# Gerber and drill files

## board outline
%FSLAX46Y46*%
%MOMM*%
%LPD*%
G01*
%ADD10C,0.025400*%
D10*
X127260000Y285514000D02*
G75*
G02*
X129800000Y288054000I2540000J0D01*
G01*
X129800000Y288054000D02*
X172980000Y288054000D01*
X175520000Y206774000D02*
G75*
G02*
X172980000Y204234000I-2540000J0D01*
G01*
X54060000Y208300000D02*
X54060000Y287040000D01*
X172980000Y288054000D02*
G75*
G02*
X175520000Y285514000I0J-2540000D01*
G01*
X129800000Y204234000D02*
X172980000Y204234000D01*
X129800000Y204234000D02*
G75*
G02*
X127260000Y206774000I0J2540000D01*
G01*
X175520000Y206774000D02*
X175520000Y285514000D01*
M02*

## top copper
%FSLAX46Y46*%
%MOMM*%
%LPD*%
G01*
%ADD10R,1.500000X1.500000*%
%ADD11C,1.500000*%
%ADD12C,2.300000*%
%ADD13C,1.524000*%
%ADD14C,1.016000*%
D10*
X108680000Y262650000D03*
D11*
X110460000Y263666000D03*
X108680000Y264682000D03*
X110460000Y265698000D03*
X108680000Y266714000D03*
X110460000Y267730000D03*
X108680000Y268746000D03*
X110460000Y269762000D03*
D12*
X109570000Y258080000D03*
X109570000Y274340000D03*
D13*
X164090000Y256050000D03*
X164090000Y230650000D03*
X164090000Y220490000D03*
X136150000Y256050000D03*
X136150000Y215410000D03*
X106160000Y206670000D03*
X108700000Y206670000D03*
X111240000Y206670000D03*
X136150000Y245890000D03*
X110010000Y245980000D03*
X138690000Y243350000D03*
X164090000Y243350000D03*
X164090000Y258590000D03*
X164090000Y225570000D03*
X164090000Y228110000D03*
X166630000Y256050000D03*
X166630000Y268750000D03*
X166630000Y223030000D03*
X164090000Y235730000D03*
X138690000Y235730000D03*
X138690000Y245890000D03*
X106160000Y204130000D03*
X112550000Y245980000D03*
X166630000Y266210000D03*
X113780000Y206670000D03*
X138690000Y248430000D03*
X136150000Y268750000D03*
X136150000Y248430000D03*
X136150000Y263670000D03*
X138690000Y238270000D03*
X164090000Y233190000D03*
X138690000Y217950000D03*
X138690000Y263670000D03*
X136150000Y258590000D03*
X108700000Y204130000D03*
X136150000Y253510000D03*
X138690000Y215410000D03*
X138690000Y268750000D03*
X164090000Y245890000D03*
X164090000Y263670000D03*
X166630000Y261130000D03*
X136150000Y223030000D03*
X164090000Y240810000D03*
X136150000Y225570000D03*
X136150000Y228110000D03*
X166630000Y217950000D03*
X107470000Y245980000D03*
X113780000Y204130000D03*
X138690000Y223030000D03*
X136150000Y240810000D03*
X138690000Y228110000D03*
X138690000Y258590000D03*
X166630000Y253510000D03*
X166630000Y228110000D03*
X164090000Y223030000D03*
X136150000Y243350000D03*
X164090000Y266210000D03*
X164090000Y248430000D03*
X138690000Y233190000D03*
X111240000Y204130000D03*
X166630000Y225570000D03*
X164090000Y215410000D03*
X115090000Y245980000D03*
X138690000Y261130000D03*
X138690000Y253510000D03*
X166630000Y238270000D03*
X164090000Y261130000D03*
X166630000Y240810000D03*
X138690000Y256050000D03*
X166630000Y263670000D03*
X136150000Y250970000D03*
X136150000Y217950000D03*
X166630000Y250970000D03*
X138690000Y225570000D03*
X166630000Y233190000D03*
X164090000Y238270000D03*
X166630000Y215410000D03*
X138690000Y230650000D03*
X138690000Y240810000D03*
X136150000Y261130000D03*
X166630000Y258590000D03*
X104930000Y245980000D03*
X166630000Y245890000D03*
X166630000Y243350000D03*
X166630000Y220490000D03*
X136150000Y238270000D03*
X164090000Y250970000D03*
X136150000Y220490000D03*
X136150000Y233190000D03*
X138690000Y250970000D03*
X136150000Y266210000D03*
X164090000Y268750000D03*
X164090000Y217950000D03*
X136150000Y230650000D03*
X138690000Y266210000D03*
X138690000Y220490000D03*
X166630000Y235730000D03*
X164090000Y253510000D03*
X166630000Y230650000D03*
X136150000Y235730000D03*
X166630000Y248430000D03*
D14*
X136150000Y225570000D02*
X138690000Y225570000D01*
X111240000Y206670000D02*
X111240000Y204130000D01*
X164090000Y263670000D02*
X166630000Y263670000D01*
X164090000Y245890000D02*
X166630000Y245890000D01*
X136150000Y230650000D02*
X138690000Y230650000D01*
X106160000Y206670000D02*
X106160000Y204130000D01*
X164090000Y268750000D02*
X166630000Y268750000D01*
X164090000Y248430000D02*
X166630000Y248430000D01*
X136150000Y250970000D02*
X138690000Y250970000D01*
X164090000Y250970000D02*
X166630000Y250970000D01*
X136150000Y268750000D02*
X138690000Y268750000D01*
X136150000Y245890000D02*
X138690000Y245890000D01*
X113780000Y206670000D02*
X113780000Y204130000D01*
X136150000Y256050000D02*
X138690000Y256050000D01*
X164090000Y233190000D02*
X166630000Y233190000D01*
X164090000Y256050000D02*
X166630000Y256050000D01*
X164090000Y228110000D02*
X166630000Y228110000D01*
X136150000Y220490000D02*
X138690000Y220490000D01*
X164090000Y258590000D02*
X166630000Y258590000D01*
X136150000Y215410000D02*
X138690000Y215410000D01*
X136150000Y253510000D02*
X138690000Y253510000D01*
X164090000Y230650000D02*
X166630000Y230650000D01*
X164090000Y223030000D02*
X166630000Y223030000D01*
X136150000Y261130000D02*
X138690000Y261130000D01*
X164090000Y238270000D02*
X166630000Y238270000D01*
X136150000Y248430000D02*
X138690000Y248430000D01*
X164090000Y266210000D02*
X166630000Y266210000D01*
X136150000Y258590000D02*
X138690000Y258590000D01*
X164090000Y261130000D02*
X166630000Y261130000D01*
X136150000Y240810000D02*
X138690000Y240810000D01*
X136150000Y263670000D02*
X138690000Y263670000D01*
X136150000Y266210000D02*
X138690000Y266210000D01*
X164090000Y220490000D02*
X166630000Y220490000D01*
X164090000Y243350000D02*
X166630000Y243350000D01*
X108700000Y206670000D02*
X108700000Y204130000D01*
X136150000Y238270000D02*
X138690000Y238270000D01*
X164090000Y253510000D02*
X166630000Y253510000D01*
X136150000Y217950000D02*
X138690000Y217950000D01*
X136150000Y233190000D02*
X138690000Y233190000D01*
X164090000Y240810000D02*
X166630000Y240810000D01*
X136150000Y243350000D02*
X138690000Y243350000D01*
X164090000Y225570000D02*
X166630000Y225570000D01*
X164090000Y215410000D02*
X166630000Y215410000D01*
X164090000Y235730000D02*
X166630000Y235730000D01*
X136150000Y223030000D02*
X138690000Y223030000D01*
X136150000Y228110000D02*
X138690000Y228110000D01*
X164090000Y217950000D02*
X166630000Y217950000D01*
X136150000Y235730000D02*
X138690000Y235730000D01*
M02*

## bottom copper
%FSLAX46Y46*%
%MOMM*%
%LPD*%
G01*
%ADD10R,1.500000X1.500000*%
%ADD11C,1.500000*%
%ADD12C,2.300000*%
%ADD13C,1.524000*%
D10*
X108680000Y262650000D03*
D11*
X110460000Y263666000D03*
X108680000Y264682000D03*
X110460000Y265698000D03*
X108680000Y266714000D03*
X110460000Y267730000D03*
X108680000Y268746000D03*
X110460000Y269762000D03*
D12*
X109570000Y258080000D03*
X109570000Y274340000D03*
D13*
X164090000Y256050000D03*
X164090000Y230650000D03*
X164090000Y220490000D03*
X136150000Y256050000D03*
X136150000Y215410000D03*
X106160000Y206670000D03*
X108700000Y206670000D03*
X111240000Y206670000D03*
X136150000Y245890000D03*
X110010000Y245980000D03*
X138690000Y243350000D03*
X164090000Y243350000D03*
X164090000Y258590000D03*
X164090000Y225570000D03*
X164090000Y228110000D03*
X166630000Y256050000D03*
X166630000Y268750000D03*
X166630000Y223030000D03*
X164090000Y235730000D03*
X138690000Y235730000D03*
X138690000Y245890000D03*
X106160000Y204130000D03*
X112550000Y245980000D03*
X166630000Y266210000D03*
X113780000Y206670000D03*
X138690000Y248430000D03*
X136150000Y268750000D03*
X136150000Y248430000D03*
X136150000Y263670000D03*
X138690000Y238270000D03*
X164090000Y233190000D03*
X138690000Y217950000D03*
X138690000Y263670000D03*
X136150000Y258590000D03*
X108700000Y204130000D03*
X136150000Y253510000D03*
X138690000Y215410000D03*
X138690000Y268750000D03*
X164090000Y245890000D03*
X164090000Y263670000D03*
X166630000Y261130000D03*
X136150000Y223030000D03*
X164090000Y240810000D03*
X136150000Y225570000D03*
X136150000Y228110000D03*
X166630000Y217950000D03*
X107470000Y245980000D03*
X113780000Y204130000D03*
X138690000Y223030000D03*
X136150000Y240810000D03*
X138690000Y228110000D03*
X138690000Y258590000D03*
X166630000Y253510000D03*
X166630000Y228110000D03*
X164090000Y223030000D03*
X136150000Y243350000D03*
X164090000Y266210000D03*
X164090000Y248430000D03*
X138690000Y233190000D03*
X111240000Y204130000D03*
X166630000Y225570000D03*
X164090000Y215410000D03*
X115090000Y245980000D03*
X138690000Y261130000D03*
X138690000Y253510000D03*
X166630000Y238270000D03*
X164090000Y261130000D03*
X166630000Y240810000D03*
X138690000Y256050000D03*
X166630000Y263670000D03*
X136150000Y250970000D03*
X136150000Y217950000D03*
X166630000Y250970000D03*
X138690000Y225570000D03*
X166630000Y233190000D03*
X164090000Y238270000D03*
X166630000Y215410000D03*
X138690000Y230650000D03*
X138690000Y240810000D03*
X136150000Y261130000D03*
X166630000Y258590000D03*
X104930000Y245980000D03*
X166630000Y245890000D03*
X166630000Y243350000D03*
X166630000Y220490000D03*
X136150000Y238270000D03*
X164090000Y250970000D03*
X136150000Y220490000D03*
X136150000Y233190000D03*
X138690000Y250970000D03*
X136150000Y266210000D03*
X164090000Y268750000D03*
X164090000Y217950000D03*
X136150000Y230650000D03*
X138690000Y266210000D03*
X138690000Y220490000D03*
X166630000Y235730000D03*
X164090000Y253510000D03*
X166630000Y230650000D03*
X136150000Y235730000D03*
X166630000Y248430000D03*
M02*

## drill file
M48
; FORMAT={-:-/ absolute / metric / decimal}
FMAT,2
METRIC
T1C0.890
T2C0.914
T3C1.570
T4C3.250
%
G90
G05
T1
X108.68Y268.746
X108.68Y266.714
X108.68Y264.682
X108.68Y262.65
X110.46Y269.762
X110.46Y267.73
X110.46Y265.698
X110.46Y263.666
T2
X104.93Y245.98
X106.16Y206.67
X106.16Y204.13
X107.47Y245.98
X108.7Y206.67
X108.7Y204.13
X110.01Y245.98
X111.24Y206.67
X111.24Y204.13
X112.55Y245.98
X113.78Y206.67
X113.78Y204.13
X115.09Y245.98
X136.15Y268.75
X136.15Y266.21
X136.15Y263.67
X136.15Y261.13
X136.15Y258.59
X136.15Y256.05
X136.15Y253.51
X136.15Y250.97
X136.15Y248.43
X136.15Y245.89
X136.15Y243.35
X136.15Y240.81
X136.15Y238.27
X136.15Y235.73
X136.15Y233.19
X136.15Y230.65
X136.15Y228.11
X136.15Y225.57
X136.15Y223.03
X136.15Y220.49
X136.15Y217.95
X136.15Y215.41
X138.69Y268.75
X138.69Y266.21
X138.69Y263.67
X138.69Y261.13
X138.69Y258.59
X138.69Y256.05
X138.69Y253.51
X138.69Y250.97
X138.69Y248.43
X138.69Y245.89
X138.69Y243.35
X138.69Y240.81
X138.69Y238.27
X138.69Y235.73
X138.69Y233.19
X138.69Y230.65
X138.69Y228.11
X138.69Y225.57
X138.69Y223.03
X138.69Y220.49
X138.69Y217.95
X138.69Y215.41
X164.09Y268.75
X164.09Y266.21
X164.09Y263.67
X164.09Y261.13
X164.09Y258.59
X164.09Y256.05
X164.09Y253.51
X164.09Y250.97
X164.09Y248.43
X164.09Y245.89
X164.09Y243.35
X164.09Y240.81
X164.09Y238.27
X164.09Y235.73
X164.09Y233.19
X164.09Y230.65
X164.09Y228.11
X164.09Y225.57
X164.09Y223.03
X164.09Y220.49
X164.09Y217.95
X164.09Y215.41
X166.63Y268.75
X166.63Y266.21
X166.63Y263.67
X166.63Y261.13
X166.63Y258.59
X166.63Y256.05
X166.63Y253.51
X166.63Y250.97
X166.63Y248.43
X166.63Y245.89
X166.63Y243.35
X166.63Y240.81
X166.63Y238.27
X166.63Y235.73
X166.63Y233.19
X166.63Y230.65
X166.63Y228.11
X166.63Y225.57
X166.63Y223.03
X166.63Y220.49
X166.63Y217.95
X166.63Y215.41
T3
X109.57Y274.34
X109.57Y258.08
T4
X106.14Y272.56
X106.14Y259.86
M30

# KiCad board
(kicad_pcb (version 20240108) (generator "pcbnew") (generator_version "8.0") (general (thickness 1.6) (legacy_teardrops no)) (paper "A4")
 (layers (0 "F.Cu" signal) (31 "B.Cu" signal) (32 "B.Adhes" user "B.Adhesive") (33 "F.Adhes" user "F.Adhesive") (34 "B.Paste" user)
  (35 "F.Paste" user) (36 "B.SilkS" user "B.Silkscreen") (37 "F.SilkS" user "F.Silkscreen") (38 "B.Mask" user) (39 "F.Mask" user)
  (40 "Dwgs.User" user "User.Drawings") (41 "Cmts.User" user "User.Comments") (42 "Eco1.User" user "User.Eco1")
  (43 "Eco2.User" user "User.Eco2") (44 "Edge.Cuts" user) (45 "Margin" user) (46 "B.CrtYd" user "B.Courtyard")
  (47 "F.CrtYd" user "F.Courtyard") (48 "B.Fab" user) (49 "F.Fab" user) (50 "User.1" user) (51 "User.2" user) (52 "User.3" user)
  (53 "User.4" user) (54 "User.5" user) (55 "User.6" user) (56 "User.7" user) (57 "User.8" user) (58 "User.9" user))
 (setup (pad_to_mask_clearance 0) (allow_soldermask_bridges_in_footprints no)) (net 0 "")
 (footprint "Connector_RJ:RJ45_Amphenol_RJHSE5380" (layer "F.Cu") (at 108.68 -262.65 90)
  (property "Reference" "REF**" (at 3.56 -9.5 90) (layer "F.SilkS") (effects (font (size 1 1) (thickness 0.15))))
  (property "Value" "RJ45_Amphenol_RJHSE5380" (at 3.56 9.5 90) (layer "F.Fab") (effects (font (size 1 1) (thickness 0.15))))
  (pad "" np_thru_hole circle (at -2.79 -2.54 90) (size 3.25 3.25) (drill 3.25) (layers "*.Cu" "*.Mask"))
  (pad "" np_thru_hole circle (at 9.91 -2.54 90) (size 3.25 3.25) (drill 3.25) (layers "*.Cu" "*.Mask"))
  (pad "1" thru_hole rect (at 0 0 90) (size 1.5 1.5) (drill 0.89) (layers "*.Cu" "*.Mask") (remove_unused_layers no))
  (pad "2" thru_hole circle (at 1.016 1.78 90) (size 1.5 1.5) (drill 0.89) (layers "*.Cu" "*.Mask") (remove_unused_layers no))
  (pad "3" thru_hole circle (at 2.032 0 90) (size 1.5 1.5) (drill 0.89) (layers "*.Cu" "*.Mask") (remove_unused_layers no))
  (pad "4" thru_hole circle (at 3.048 1.78 90) (size 1.5 1.5) (drill 0.89) (layers "*.Cu" "*.Mask") (remove_unused_layers no))
  (pad "5" thru_hole circle (at 4.064 0 90) (size 1.5 1.5) (drill 0.89) (layers "*.Cu" "*.Mask") (remove_unused_layers no))
  (pad "6" thru_hole circle (at 5.08 1.78 90) (size 1.5 1.5) (drill 0.89) (layers "*.Cu" "*.Mask") (remove_unused_layers no))
  (pad "7" thru_hole circle (at 6.096 0 90) (size 1.5 1.5) (drill 0.89) (layers "*.Cu" "*.Mask") (remove_unused_layers no))
  (pad "8" thru_hole circle (at 7.112 1.78 90) (size 1.5 1.5) (drill 0.89) (layers "*.Cu" "*.Mask") (remove_unused_layers no))
  (pad "SH" thru_hole circle (at -4.57 0.89 90) (size 2.3 2.3) (drill 1.57) (layers "*.Cu" "*.Mask") (remove_unused_layers no))
  (pad "SH" thru_hole circle (at 11.69 0.89 90) (size 2.3 2.3) (drill 1.57) (layers "*.Cu" "*.Mask") (remove_unused_layers no)))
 (gr_arc (start 127.26 -285.514) (mid 128.003949 -287.310051) (end 129.8 -288.054) (stroke (width 0.0254) (type default))
  (layer "Edge.Cuts"))
 (gr_line (start 129.8 -288.054) (end 172.98 -288.054) (stroke (width 0.0254) (type default)) (layer "Edge.Cuts"))
 (gr_arc (start 175.52 -206.774) (mid 174.776051 -204.977949) (end 172.98 -204.234) (stroke (width 0.0254) (type default))
  (layer "Edge.Cuts"))
 (gr_line (start 54.06 -208.3) (end 54.06 -287.04) (stroke (width 0.0254) (type solid)) (layer "Edge.Cuts"))
 (gr_arc (start 172.98 -288.054) (mid 174.776051 -287.310051) (end 175.52 -285.514) (stroke (width 0.0254) (type default))
  (layer "Edge.Cuts"))
 (gr_line (start 129.8 -204.234) (end 172.98 -204.234) (stroke (width 0.0254) (type default)) (layer "Edge.Cuts"))
 (gr_arc (start 129.8 -204.234) (mid 128.003949 -204.977949) (end 127.26 -206.774) (stroke (width 0.0254) (type default))
  (layer "Edge.Cuts"))
 (gr_line (start 175.52 -206.774) (end 175.52 -285.514) (stroke (width 0.0254) (type solid)) (layer "Edge.Cuts"))
 (segment (start 136.15 -225.57) (end 138.69 -225.57) (width 1.016) (layer "F.Cu") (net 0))
 (segment (start 111.24 -206.67) (end 111.24 -204.13) (width 1.016) (layer "F.Cu") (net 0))
 (segment (start 164.09 -263.67) (end 166.63 -263.67) (width 1.016) (layer "F.Cu") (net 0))
 (segment (start 164.09 -245.89) (end 166.63 -245.89) (width 1.016) (layer "F.Cu") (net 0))
 (segment (start 136.15 -230.65) (end 138.69 -230.65) (width 1.016) (layer "F.Cu") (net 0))
 (segment (start 106.16 -206.67) (end 106.16 -204.13) (width 1.016) (layer "F.Cu") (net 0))
 (segment (start 164.09 -268.75) (end 166.63 -268.75) (width 1.016) (layer "F.Cu") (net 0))
 (segment (start 164.09 -248.43) (end 166.63 -248.43) (width 1.016) (layer "F.Cu") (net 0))
 (segment (start 136.15 -250.97) (end 138.69 -250.97) (width 1.016) (layer "F.Cu") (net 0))
 (segment (start 164.09 -250.97) (end 166.63 -250.97) (width 1.016) (layer "F.Cu") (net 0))
 (segment (start 136.15 -268.75) (end 138.69 -268.75) (width 1.016) (layer "F.Cu") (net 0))
 (segment (start 136.15 -245.89) (end 138.69 -245.89) (width 1.016) (layer "F.Cu") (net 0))
 (segment (start 113.78 -206.67) (end 113.78 -204.13) (width 1.016) (layer "F.Cu") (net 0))
 (segment (start 136.15 -256.05) (end 138.69 -256.05) (width 1.016) (layer "F.Cu") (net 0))
 (segment (start 164.09 -233.19) (end 166.63 -233.19) (width 1.016) (layer "F.Cu") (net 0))
 (segment (start 164.09 -256.05) (end 166.63 -256.05) (width 1.016) (layer "F.Cu") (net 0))
 (segment (start 164.09 -228.11) (end 166.63 -228.11) (width 1.016) (layer "F.Cu") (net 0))
 (segment (start 136.15 -220.49) (end 138.69 -220.49) (width 1.016) (layer "F.Cu") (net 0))
 (segment (start 164.09 -258.59) (end 166.63 -258.59) (width 1.016) (layer "F.Cu") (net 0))
 (segment (start 136.15 -215.41) (end 138.69 -215.41) (width 1.016) (layer "F.Cu") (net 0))
 (segment (start 136.15 -253.51) (end 138.69 -253.51) (width 1.016) (layer "F.Cu") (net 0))
 (segment (start 164.09 -230.65) (end 166.63 -230.65) (width 1.016) (layer "F.Cu") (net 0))
 (segment (start 164.09 -223.03) (end 166.63 -223.03) (width 1.016) (layer "F.Cu") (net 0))
 (segment (start 136.15 -261.13) (end 138.69 -261.13) (width 1.016) (layer "F.Cu") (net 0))
 (segment (start 164.09 -238.27) (end 166.63 -238.27) (width 1.016) (layer "F.Cu") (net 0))
 (segment (start 136.15 -248.43) (end 138.69 -248.43) (width 1.016) (layer "F.Cu") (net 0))
 (segment (start 164.09 -266.21) (end 166.63 -266.21) (width 1.016) (layer "F.Cu") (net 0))
 (segment (start 136.15 -258.59) (end 138.69 -258.59) (width 1.016) (layer "F.Cu") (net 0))
 (segment (start 164.09 -261.13) (end 166.63 -261.13) (width 1.016) (layer "F.Cu") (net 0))
 (segment (start 136.15 -240.81) (end 138.69 -240.81) (width 1.016) (layer "F.Cu") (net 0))
 (segment (start 136.15 -263.67) (end 138.69 -263.67) (width 1.016) (layer "F.Cu") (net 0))
 (segment (start 136.15 -266.21) (end 138.69 -266.21) (width 1.016) (layer "F.Cu") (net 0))
 (segment (start 164.09 -220.49) (end 166.63 -220.49) (width 1.016) (layer "F.Cu") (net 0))
 (segment (start 164.09 -243.35) (end 166.63 -243.35) (width 1.016) (layer "F.Cu") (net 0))
 (segment (start 108.7 -206.67) (end 108.7 -204.13) (width 1.016) (layer "F.Cu") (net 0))
 (segment (start 136.15 -238.27) (end 138.69 -238.27) (width 1.016) (layer "F.Cu") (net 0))
 (segment (start 164.09 -253.51) (end 166.63 -253.51) (width 1.016) (layer "F.Cu") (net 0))
 (segment (start 136.15 -217.95) (end 138.69 -217.95) (width 1.016) (layer "F.Cu") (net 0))
 (segment (start 136.15 -233.19) (end 138.69 -233.19) (width 1.016) (layer "F.Cu") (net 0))
 (segment (start 164.09 -240.81) (end 166.63 -240.81) (width 1.016) (layer "F.Cu") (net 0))
 (segment (start 136.15 -243.35) (end 138.69 -243.35) (width 1.016) (layer "F.Cu") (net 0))
 (segment (start 164.09 -225.57) (end 166.63 -225.57) (width 1.016) (layer "F.Cu") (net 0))
 (segment (start 164.09 -215.41) (end 166.63 -215.41) (width 1.016) (layer "F.Cu") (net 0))
 (segment (start 164.09 -235.73) (end 166.63 -235.73) (width 1.016) (layer "F.Cu") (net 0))
 (segment (start 136.15 -223.03) (end 138.69 -223.03) (width 1.016) (layer "F.Cu") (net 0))
 (segment (start 136.15 -228.11) (end 138.69 -228.11) (width 1.016) (layer "F.Cu") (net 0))
 (segment (start 164.09 -217.95) (end 166.63 -217.95) (width 1.016) (layer "F.Cu") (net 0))
 (segment (start 136.15 -235.73) (end 138.69 -235.73) (width 1.016) (layer "F.Cu") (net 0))
 (via (at 164.09 -256.05) (size 1.524) (drill 0.9144) (layers "F.Cu" "B.Cu") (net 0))
 (via (at 164.09 -230.65) (size 1.524) (drill 0.9144) (layers "F.Cu" "B.Cu") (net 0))
 (via (at 164.09 -220.49) (size 1.524) (drill 0.9144) (layers "F.Cu" "B.Cu") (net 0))
 (via (at 136.15 -256.05) (size 1.524) (drill 0.9144) (layers "F.Cu" "B.Cu") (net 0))
 (via (at 136.15 -215.41) (size 1.524) (drill 0.9144) (layers "F.Cu" "B.Cu") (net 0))
 (via (at 106.16 -206.67) (size 1.524) (drill 0.9144) (layers "F.Cu" "B.Cu") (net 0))
 (via (at 108.7 -206.67) (size 1.524) (drill 0.9144) (layers "F.Cu" "B.Cu") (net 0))
 (via (at 111.24 -206.67) (size 1.524) (drill 0.9144) (layers "F.Cu" "B.Cu") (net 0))
 (via (at 136.15 -245.89) (size 1.524) (drill 0.9144) (layers "F.Cu" "B.Cu") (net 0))
 (via (at 110.01 -245.98) (size 1.524) (drill 0.9144) (layers "F.Cu" "B.Cu") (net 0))
 (via (at 138.69 -243.35) (size 1.524) (drill 0.9144) (layers "F.Cu" "B.Cu") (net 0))
 (via (at 164.09 -243.35) (size 1.524) (drill 0.9144) (layers "F.Cu" "B.Cu") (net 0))
 (via (at 164.09 -258.59) (size 1.524) (drill 0.9144) (layers "F.Cu" "B.Cu") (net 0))
 (via (at 164.09 -225.57) (size 1.524) (drill 0.9144) (layers "F.Cu" "B.Cu") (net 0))
 (via (at 164.09 -228.11) (size 1.524) (drill 0.9144) (layers "F.Cu" "B.Cu") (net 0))
 (via (at 166.63 -256.05) (size 1.524) (drill 0.9144) (layers "F.Cu" "B.Cu") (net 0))
 (via (at 166.63 -268.75) (size 1.524) (drill 0.9144) (layers "F.Cu" "B.Cu") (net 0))
 (via (at 166.63 -223.03) (size 1.524) (drill 0.9144) (layers "F.Cu" "B.Cu") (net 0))
 (via (at 164.09 -235.73) (size 1.524) (drill 0.9144) (layers "F.Cu" "B.Cu") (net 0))
 (via (at 138.69 -235.73) (size 1.524) (drill 0.9144) (layers "F.Cu" "B.Cu") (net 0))
 (via (at 138.69 -245.89) (size 1.524) (drill 0.9144) (layers "F.Cu" "B.Cu") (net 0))
 (via (at 106.16 -204.13) (size 1.524) (drill 0.9144) (layers "F.Cu" "B.Cu") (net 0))
 (via (at 112.55 -245.98) (size 1.524) (drill 0.9144) (layers "F.Cu" "B.Cu") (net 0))
 (via (at 166.63 -266.21) (size 1.524) (drill 0.9144) (layers "F.Cu" "B.Cu") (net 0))
 (via (at 113.78 -206.67) (size 1.524) (drill 0.9144) (layers "F.Cu" "B.Cu") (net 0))
 (via (at 138.69 -248.43) (size 1.524) (drill 0.9144) (layers "F.Cu" "B.Cu") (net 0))
 (via (at 136.15 -268.75) (size 1.524) (drill 0.9144) (layers "F.Cu" "B.Cu") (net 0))
 (via (at 136.15 -248.43) (size 1.524) (drill 0.9144) (layers "F.Cu" "B.Cu") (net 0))
 (via (at 136.15 -263.67) (size 1.524) (drill 0.9144) (layers "F.Cu" "B.Cu") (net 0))
 (via (at 138.69 -238.27) (size 1.524) (drill 0.9144) (layers "F.Cu" "B.Cu") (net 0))
 (via (at 164.09 -233.19) (size 1.524) (drill 0.9144) (layers "F.Cu" "B.Cu") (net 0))
 (via (at 138.69 -217.95) (size 1.524) (drill 0.9144) (layers "F.Cu" "B.Cu") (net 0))
 (via (at 138.69 -263.67) (size 1.524) (drill 0.9144) (layers "F.Cu" "B.Cu") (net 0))
 (via (at 136.15 -258.59) (size 1.524) (drill 0.9144) (layers "F.Cu" "B.Cu") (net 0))
 (via (at 108.7 -204.13) (size 1.524) (drill 0.9144) (layers "F.Cu" "B.Cu") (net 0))
 (via (at 136.15 -253.51) (size 1.524) (drill 0.9144) (layers "F.Cu" "B.Cu") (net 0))
 (via (at 138.69 -215.41) (size 1.524) (drill 0.9144) (layers "F.Cu" "B.Cu") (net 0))
 (via (at 138.69 -268.75) (size 1.524) (drill 0.9144) (layers "F.Cu" "B.Cu") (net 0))
 (via (at 164.09 -245.89) (size 1.524) (drill 0.9144) (layers "F.Cu" "B.Cu") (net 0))
 (via (at 164.09 -263.67) (size 1.524) (drill 0.9144) (layers "F.Cu" "B.Cu") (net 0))
 (via (at 166.63 -261.13) (size 1.524) (drill 0.9144) (layers "F.Cu" "B.Cu") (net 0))
 (via (at 136.15 -223.03) (size 1.524) (drill 0.9144) (layers "F.Cu" "B.Cu") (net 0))
 (via (at 164.09 -240.81) (size 1.524) (drill 0.9144) (layers "F.Cu" "B.Cu") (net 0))
 (via (at 136.15 -225.57) (size 1.524) (drill 0.9144) (layers "F.Cu" "B.Cu") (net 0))
 (via (at 136.15 -228.11) (size 1.524) (drill 0.9144) (layers "F.Cu" "B.Cu") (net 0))
 (via (at 166.63 -217.95) (size 1.524) (drill 0.9144) (layers "F.Cu" "B.Cu") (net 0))
 (via (at 107.47 -245.98) (size 1.524) (drill 0.9144) (layers "F.Cu" "B.Cu") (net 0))
 (via (at 113.78 -204.13) (size 1.524) (drill 0.9144) (layers "F.Cu" "B.Cu") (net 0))
 (via (at 138.69 -223.03) (size 1.524) (drill 0.9144) (layers "F.Cu" "B.Cu") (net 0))
 (via (at 136.15 -240.81) (size 1.524) (drill 0.9144) (layers "F.Cu" "B.Cu") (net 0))
 (via (at 138.69 -228.11) (size 1.524) (drill 0.9144) (layers "F.Cu" "B.Cu") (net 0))
 (via (at 138.69 -258.59) (size 1.524) (drill 0.9144) (layers "F.Cu" "B.Cu") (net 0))
 (via (at 166.63 -253.51) (size 1.524) (drill 0.9144) (layers "F.Cu" "B.Cu") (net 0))
 (via (at 166.63 -228.11) (size 1.524) (drill 0.9144) (layers "F.Cu" "B.Cu") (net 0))
 (via (at 164.09 -223.03) (size 1.524) (drill 0.9144) (layers "F.Cu" "B.Cu") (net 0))
 (via (at 136.15 -243.35) (size 1.524) (drill 0.9144) (layers "F.Cu" "B.Cu") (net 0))
 (via (at 164.09 -266.21) (size 1.524) (drill 0.9144) (layers "F.Cu" "B.Cu") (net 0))
 (via (at 164.09 -248.43) (size 1.524) (drill 0.9144) (layers "F.Cu" "B.Cu") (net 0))
 (via (at 138.69 -233.19) (size 1.524) (drill 0.9144) (layers "F.Cu" "B.Cu") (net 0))
 (via (at 111.24 -204.13) (size 1.524) (drill 0.9144) (layers "F.Cu" "B.Cu") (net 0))
 (via (at 166.63 -225.57) (size 1.524) (drill 0.9144) (layers "F.Cu" "B.Cu") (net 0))
 (via (at 164.09 -215.41) (size 1.524) (drill 0.9144) (layers "F.Cu" "B.Cu") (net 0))
 (via (at 115.09 -245.98) (size 1.524) (drill 0.9144) (layers "F.Cu" "B.Cu") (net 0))
 (via (at 138.69 -261.13) (size 1.524) (drill 0.9144) (layers "F.Cu" "B.Cu") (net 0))
 (via (at 138.69 -253.51) (size 1.524) (drill 0.9144) (layers "F.Cu" "B.Cu") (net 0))
 (via (at 166.63 -238.27) (size 1.524) (drill 0.9144) (layers "F.Cu" "B.Cu") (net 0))
 (via (at 164.09 -261.13) (size 1.524) (drill 0.9144) (layers "F.Cu" "B.Cu") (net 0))
 (via (at 166.63 -240.81) (size 1.524) (drill 0.9144) (layers "F.Cu" "B.Cu") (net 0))
 (via (at 138.69 -256.05) (size 1.524) (drill 0.9144) (layers "F.Cu" "B.Cu") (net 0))
 (via (at 166.63 -263.67) (size 1.524) (drill 0.9144) (layers "F.Cu" "B.Cu") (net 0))
 (via (at 136.15 -250.97) (size 1.524) (drill 0.9144) (layers "F.Cu" "B.Cu") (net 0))
 (via (at 136.15 -217.95) (size 1.524) (drill 0.9144) (layers "F.Cu" "B.Cu") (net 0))
 (via (at 166.63 -250.97) (size 1.524) (drill 0.9144) (layers "F.Cu" "B.Cu") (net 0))
 (via (at 138.69 -225.57) (size 1.524) (drill 0.9144) (layers "F.Cu" "B.Cu") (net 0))
 (via (at 166.63 -233.19) (size 1.524) (drill 0.9144) (layers "F.Cu" "B.Cu") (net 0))
 (via (at 164.09 -238.27) (size 1.524) (drill 0.9144) (layers "F.Cu" "B.Cu") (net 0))
 (via (at 166.63 -215.41) (size 1.524) (drill 0.9144) (layers "F.Cu" "B.Cu") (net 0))
 (via (at 138.69 -230.65) (size 1.524) (drill 0.9144) (layers "F.Cu" "B.Cu") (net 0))
 (via (at 138.69 -240.81) (size 1.524) (drill 0.9144) (layers "F.Cu" "B.Cu") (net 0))
 (via (at 136.15 -261.13) (size 1.524) (drill 0.9144) (layers "F.Cu" "B.Cu") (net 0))
 (via (at 166.63 -258.59) (size 1.524) (drill 0.9144) (layers "F.Cu" "B.Cu") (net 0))
 (via (at 104.93 -245.98) (size 1.524) (drill 0.9144) (layers "F.Cu" "B.Cu") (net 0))
 (via (at 166.63 -245.89) (size 1.524) (drill 0.9144) (layers "F.Cu" "B.Cu") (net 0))
 (via (at 166.63 -243.35) (size 1.524) (drill 0.9144) (layers "F.Cu" "B.Cu") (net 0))
 (via (at 166.63 -220.49) (size 1.524) (drill 0.9144) (layers "F.Cu" "B.Cu") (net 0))
 (via (at 136.15 -238.27) (size 1.524) (drill 0.9144) (layers "F.Cu" "B.Cu") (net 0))
 (via (at 164.09 -250.97) (size 1.524) (drill 0.9144) (layers "F.Cu" "B.Cu") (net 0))
 (via (at 136.15 -220.49) (size 1.524) (drill 0.9144) (layers "F.Cu" "B.Cu") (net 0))
 (via (at 136.15 -233.19) (size 1.524) (drill 0.9144) (layers "F.Cu" "B.Cu") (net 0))
 (via (at 138.69 -250.97) (size 1.524) (drill 0.9144) (layers "F.Cu" "B.Cu") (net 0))
 (via (at 136.15 -266.21) (size 1.524) (drill 0.9144) (layers "F.Cu" "B.Cu") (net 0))
 (via (at 164.09 -268.75) (size 1.524) (drill 0.9144) (layers "F.Cu" "B.Cu") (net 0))
 (via (at 164.09 -217.95) (size 1.524) (drill 0.9144) (layers "F.Cu" "B.Cu") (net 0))
 (via (at 136.15 -230.65) (size 1.524) (drill 0.9144) (layers "F.Cu" "B.Cu") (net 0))
 (via (at 138.69 -266.21) (size 1.524) (drill 0.9144) (layers "F.Cu" "B.Cu") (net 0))
 (via (at 138.69 -220.49) (size 1.524) (drill 0.9144) (layers "F.Cu" "B.Cu") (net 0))
 (via (at 166.63 -235.73) (size 1.524) (drill 0.9144) (layers "F.Cu" "B.Cu") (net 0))
 (via (at 164.09 -253.51) (size 1.524) (drill 0.9144) (layers "F.Cu" "B.Cu") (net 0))
 (via (at 166.63 -230.65) (size 1.524) (drill 0.9144) (layers "F.Cu" "B.Cu") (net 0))
 (via (at 136.15 -235.73) (size 1.524) (drill 0.9144) (layers "F.Cu" "B.Cu") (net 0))
 (via (at 166.63 -248.43) (size 1.524) (drill 0.9144) (layers "F.Cu" "B.Cu") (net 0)))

